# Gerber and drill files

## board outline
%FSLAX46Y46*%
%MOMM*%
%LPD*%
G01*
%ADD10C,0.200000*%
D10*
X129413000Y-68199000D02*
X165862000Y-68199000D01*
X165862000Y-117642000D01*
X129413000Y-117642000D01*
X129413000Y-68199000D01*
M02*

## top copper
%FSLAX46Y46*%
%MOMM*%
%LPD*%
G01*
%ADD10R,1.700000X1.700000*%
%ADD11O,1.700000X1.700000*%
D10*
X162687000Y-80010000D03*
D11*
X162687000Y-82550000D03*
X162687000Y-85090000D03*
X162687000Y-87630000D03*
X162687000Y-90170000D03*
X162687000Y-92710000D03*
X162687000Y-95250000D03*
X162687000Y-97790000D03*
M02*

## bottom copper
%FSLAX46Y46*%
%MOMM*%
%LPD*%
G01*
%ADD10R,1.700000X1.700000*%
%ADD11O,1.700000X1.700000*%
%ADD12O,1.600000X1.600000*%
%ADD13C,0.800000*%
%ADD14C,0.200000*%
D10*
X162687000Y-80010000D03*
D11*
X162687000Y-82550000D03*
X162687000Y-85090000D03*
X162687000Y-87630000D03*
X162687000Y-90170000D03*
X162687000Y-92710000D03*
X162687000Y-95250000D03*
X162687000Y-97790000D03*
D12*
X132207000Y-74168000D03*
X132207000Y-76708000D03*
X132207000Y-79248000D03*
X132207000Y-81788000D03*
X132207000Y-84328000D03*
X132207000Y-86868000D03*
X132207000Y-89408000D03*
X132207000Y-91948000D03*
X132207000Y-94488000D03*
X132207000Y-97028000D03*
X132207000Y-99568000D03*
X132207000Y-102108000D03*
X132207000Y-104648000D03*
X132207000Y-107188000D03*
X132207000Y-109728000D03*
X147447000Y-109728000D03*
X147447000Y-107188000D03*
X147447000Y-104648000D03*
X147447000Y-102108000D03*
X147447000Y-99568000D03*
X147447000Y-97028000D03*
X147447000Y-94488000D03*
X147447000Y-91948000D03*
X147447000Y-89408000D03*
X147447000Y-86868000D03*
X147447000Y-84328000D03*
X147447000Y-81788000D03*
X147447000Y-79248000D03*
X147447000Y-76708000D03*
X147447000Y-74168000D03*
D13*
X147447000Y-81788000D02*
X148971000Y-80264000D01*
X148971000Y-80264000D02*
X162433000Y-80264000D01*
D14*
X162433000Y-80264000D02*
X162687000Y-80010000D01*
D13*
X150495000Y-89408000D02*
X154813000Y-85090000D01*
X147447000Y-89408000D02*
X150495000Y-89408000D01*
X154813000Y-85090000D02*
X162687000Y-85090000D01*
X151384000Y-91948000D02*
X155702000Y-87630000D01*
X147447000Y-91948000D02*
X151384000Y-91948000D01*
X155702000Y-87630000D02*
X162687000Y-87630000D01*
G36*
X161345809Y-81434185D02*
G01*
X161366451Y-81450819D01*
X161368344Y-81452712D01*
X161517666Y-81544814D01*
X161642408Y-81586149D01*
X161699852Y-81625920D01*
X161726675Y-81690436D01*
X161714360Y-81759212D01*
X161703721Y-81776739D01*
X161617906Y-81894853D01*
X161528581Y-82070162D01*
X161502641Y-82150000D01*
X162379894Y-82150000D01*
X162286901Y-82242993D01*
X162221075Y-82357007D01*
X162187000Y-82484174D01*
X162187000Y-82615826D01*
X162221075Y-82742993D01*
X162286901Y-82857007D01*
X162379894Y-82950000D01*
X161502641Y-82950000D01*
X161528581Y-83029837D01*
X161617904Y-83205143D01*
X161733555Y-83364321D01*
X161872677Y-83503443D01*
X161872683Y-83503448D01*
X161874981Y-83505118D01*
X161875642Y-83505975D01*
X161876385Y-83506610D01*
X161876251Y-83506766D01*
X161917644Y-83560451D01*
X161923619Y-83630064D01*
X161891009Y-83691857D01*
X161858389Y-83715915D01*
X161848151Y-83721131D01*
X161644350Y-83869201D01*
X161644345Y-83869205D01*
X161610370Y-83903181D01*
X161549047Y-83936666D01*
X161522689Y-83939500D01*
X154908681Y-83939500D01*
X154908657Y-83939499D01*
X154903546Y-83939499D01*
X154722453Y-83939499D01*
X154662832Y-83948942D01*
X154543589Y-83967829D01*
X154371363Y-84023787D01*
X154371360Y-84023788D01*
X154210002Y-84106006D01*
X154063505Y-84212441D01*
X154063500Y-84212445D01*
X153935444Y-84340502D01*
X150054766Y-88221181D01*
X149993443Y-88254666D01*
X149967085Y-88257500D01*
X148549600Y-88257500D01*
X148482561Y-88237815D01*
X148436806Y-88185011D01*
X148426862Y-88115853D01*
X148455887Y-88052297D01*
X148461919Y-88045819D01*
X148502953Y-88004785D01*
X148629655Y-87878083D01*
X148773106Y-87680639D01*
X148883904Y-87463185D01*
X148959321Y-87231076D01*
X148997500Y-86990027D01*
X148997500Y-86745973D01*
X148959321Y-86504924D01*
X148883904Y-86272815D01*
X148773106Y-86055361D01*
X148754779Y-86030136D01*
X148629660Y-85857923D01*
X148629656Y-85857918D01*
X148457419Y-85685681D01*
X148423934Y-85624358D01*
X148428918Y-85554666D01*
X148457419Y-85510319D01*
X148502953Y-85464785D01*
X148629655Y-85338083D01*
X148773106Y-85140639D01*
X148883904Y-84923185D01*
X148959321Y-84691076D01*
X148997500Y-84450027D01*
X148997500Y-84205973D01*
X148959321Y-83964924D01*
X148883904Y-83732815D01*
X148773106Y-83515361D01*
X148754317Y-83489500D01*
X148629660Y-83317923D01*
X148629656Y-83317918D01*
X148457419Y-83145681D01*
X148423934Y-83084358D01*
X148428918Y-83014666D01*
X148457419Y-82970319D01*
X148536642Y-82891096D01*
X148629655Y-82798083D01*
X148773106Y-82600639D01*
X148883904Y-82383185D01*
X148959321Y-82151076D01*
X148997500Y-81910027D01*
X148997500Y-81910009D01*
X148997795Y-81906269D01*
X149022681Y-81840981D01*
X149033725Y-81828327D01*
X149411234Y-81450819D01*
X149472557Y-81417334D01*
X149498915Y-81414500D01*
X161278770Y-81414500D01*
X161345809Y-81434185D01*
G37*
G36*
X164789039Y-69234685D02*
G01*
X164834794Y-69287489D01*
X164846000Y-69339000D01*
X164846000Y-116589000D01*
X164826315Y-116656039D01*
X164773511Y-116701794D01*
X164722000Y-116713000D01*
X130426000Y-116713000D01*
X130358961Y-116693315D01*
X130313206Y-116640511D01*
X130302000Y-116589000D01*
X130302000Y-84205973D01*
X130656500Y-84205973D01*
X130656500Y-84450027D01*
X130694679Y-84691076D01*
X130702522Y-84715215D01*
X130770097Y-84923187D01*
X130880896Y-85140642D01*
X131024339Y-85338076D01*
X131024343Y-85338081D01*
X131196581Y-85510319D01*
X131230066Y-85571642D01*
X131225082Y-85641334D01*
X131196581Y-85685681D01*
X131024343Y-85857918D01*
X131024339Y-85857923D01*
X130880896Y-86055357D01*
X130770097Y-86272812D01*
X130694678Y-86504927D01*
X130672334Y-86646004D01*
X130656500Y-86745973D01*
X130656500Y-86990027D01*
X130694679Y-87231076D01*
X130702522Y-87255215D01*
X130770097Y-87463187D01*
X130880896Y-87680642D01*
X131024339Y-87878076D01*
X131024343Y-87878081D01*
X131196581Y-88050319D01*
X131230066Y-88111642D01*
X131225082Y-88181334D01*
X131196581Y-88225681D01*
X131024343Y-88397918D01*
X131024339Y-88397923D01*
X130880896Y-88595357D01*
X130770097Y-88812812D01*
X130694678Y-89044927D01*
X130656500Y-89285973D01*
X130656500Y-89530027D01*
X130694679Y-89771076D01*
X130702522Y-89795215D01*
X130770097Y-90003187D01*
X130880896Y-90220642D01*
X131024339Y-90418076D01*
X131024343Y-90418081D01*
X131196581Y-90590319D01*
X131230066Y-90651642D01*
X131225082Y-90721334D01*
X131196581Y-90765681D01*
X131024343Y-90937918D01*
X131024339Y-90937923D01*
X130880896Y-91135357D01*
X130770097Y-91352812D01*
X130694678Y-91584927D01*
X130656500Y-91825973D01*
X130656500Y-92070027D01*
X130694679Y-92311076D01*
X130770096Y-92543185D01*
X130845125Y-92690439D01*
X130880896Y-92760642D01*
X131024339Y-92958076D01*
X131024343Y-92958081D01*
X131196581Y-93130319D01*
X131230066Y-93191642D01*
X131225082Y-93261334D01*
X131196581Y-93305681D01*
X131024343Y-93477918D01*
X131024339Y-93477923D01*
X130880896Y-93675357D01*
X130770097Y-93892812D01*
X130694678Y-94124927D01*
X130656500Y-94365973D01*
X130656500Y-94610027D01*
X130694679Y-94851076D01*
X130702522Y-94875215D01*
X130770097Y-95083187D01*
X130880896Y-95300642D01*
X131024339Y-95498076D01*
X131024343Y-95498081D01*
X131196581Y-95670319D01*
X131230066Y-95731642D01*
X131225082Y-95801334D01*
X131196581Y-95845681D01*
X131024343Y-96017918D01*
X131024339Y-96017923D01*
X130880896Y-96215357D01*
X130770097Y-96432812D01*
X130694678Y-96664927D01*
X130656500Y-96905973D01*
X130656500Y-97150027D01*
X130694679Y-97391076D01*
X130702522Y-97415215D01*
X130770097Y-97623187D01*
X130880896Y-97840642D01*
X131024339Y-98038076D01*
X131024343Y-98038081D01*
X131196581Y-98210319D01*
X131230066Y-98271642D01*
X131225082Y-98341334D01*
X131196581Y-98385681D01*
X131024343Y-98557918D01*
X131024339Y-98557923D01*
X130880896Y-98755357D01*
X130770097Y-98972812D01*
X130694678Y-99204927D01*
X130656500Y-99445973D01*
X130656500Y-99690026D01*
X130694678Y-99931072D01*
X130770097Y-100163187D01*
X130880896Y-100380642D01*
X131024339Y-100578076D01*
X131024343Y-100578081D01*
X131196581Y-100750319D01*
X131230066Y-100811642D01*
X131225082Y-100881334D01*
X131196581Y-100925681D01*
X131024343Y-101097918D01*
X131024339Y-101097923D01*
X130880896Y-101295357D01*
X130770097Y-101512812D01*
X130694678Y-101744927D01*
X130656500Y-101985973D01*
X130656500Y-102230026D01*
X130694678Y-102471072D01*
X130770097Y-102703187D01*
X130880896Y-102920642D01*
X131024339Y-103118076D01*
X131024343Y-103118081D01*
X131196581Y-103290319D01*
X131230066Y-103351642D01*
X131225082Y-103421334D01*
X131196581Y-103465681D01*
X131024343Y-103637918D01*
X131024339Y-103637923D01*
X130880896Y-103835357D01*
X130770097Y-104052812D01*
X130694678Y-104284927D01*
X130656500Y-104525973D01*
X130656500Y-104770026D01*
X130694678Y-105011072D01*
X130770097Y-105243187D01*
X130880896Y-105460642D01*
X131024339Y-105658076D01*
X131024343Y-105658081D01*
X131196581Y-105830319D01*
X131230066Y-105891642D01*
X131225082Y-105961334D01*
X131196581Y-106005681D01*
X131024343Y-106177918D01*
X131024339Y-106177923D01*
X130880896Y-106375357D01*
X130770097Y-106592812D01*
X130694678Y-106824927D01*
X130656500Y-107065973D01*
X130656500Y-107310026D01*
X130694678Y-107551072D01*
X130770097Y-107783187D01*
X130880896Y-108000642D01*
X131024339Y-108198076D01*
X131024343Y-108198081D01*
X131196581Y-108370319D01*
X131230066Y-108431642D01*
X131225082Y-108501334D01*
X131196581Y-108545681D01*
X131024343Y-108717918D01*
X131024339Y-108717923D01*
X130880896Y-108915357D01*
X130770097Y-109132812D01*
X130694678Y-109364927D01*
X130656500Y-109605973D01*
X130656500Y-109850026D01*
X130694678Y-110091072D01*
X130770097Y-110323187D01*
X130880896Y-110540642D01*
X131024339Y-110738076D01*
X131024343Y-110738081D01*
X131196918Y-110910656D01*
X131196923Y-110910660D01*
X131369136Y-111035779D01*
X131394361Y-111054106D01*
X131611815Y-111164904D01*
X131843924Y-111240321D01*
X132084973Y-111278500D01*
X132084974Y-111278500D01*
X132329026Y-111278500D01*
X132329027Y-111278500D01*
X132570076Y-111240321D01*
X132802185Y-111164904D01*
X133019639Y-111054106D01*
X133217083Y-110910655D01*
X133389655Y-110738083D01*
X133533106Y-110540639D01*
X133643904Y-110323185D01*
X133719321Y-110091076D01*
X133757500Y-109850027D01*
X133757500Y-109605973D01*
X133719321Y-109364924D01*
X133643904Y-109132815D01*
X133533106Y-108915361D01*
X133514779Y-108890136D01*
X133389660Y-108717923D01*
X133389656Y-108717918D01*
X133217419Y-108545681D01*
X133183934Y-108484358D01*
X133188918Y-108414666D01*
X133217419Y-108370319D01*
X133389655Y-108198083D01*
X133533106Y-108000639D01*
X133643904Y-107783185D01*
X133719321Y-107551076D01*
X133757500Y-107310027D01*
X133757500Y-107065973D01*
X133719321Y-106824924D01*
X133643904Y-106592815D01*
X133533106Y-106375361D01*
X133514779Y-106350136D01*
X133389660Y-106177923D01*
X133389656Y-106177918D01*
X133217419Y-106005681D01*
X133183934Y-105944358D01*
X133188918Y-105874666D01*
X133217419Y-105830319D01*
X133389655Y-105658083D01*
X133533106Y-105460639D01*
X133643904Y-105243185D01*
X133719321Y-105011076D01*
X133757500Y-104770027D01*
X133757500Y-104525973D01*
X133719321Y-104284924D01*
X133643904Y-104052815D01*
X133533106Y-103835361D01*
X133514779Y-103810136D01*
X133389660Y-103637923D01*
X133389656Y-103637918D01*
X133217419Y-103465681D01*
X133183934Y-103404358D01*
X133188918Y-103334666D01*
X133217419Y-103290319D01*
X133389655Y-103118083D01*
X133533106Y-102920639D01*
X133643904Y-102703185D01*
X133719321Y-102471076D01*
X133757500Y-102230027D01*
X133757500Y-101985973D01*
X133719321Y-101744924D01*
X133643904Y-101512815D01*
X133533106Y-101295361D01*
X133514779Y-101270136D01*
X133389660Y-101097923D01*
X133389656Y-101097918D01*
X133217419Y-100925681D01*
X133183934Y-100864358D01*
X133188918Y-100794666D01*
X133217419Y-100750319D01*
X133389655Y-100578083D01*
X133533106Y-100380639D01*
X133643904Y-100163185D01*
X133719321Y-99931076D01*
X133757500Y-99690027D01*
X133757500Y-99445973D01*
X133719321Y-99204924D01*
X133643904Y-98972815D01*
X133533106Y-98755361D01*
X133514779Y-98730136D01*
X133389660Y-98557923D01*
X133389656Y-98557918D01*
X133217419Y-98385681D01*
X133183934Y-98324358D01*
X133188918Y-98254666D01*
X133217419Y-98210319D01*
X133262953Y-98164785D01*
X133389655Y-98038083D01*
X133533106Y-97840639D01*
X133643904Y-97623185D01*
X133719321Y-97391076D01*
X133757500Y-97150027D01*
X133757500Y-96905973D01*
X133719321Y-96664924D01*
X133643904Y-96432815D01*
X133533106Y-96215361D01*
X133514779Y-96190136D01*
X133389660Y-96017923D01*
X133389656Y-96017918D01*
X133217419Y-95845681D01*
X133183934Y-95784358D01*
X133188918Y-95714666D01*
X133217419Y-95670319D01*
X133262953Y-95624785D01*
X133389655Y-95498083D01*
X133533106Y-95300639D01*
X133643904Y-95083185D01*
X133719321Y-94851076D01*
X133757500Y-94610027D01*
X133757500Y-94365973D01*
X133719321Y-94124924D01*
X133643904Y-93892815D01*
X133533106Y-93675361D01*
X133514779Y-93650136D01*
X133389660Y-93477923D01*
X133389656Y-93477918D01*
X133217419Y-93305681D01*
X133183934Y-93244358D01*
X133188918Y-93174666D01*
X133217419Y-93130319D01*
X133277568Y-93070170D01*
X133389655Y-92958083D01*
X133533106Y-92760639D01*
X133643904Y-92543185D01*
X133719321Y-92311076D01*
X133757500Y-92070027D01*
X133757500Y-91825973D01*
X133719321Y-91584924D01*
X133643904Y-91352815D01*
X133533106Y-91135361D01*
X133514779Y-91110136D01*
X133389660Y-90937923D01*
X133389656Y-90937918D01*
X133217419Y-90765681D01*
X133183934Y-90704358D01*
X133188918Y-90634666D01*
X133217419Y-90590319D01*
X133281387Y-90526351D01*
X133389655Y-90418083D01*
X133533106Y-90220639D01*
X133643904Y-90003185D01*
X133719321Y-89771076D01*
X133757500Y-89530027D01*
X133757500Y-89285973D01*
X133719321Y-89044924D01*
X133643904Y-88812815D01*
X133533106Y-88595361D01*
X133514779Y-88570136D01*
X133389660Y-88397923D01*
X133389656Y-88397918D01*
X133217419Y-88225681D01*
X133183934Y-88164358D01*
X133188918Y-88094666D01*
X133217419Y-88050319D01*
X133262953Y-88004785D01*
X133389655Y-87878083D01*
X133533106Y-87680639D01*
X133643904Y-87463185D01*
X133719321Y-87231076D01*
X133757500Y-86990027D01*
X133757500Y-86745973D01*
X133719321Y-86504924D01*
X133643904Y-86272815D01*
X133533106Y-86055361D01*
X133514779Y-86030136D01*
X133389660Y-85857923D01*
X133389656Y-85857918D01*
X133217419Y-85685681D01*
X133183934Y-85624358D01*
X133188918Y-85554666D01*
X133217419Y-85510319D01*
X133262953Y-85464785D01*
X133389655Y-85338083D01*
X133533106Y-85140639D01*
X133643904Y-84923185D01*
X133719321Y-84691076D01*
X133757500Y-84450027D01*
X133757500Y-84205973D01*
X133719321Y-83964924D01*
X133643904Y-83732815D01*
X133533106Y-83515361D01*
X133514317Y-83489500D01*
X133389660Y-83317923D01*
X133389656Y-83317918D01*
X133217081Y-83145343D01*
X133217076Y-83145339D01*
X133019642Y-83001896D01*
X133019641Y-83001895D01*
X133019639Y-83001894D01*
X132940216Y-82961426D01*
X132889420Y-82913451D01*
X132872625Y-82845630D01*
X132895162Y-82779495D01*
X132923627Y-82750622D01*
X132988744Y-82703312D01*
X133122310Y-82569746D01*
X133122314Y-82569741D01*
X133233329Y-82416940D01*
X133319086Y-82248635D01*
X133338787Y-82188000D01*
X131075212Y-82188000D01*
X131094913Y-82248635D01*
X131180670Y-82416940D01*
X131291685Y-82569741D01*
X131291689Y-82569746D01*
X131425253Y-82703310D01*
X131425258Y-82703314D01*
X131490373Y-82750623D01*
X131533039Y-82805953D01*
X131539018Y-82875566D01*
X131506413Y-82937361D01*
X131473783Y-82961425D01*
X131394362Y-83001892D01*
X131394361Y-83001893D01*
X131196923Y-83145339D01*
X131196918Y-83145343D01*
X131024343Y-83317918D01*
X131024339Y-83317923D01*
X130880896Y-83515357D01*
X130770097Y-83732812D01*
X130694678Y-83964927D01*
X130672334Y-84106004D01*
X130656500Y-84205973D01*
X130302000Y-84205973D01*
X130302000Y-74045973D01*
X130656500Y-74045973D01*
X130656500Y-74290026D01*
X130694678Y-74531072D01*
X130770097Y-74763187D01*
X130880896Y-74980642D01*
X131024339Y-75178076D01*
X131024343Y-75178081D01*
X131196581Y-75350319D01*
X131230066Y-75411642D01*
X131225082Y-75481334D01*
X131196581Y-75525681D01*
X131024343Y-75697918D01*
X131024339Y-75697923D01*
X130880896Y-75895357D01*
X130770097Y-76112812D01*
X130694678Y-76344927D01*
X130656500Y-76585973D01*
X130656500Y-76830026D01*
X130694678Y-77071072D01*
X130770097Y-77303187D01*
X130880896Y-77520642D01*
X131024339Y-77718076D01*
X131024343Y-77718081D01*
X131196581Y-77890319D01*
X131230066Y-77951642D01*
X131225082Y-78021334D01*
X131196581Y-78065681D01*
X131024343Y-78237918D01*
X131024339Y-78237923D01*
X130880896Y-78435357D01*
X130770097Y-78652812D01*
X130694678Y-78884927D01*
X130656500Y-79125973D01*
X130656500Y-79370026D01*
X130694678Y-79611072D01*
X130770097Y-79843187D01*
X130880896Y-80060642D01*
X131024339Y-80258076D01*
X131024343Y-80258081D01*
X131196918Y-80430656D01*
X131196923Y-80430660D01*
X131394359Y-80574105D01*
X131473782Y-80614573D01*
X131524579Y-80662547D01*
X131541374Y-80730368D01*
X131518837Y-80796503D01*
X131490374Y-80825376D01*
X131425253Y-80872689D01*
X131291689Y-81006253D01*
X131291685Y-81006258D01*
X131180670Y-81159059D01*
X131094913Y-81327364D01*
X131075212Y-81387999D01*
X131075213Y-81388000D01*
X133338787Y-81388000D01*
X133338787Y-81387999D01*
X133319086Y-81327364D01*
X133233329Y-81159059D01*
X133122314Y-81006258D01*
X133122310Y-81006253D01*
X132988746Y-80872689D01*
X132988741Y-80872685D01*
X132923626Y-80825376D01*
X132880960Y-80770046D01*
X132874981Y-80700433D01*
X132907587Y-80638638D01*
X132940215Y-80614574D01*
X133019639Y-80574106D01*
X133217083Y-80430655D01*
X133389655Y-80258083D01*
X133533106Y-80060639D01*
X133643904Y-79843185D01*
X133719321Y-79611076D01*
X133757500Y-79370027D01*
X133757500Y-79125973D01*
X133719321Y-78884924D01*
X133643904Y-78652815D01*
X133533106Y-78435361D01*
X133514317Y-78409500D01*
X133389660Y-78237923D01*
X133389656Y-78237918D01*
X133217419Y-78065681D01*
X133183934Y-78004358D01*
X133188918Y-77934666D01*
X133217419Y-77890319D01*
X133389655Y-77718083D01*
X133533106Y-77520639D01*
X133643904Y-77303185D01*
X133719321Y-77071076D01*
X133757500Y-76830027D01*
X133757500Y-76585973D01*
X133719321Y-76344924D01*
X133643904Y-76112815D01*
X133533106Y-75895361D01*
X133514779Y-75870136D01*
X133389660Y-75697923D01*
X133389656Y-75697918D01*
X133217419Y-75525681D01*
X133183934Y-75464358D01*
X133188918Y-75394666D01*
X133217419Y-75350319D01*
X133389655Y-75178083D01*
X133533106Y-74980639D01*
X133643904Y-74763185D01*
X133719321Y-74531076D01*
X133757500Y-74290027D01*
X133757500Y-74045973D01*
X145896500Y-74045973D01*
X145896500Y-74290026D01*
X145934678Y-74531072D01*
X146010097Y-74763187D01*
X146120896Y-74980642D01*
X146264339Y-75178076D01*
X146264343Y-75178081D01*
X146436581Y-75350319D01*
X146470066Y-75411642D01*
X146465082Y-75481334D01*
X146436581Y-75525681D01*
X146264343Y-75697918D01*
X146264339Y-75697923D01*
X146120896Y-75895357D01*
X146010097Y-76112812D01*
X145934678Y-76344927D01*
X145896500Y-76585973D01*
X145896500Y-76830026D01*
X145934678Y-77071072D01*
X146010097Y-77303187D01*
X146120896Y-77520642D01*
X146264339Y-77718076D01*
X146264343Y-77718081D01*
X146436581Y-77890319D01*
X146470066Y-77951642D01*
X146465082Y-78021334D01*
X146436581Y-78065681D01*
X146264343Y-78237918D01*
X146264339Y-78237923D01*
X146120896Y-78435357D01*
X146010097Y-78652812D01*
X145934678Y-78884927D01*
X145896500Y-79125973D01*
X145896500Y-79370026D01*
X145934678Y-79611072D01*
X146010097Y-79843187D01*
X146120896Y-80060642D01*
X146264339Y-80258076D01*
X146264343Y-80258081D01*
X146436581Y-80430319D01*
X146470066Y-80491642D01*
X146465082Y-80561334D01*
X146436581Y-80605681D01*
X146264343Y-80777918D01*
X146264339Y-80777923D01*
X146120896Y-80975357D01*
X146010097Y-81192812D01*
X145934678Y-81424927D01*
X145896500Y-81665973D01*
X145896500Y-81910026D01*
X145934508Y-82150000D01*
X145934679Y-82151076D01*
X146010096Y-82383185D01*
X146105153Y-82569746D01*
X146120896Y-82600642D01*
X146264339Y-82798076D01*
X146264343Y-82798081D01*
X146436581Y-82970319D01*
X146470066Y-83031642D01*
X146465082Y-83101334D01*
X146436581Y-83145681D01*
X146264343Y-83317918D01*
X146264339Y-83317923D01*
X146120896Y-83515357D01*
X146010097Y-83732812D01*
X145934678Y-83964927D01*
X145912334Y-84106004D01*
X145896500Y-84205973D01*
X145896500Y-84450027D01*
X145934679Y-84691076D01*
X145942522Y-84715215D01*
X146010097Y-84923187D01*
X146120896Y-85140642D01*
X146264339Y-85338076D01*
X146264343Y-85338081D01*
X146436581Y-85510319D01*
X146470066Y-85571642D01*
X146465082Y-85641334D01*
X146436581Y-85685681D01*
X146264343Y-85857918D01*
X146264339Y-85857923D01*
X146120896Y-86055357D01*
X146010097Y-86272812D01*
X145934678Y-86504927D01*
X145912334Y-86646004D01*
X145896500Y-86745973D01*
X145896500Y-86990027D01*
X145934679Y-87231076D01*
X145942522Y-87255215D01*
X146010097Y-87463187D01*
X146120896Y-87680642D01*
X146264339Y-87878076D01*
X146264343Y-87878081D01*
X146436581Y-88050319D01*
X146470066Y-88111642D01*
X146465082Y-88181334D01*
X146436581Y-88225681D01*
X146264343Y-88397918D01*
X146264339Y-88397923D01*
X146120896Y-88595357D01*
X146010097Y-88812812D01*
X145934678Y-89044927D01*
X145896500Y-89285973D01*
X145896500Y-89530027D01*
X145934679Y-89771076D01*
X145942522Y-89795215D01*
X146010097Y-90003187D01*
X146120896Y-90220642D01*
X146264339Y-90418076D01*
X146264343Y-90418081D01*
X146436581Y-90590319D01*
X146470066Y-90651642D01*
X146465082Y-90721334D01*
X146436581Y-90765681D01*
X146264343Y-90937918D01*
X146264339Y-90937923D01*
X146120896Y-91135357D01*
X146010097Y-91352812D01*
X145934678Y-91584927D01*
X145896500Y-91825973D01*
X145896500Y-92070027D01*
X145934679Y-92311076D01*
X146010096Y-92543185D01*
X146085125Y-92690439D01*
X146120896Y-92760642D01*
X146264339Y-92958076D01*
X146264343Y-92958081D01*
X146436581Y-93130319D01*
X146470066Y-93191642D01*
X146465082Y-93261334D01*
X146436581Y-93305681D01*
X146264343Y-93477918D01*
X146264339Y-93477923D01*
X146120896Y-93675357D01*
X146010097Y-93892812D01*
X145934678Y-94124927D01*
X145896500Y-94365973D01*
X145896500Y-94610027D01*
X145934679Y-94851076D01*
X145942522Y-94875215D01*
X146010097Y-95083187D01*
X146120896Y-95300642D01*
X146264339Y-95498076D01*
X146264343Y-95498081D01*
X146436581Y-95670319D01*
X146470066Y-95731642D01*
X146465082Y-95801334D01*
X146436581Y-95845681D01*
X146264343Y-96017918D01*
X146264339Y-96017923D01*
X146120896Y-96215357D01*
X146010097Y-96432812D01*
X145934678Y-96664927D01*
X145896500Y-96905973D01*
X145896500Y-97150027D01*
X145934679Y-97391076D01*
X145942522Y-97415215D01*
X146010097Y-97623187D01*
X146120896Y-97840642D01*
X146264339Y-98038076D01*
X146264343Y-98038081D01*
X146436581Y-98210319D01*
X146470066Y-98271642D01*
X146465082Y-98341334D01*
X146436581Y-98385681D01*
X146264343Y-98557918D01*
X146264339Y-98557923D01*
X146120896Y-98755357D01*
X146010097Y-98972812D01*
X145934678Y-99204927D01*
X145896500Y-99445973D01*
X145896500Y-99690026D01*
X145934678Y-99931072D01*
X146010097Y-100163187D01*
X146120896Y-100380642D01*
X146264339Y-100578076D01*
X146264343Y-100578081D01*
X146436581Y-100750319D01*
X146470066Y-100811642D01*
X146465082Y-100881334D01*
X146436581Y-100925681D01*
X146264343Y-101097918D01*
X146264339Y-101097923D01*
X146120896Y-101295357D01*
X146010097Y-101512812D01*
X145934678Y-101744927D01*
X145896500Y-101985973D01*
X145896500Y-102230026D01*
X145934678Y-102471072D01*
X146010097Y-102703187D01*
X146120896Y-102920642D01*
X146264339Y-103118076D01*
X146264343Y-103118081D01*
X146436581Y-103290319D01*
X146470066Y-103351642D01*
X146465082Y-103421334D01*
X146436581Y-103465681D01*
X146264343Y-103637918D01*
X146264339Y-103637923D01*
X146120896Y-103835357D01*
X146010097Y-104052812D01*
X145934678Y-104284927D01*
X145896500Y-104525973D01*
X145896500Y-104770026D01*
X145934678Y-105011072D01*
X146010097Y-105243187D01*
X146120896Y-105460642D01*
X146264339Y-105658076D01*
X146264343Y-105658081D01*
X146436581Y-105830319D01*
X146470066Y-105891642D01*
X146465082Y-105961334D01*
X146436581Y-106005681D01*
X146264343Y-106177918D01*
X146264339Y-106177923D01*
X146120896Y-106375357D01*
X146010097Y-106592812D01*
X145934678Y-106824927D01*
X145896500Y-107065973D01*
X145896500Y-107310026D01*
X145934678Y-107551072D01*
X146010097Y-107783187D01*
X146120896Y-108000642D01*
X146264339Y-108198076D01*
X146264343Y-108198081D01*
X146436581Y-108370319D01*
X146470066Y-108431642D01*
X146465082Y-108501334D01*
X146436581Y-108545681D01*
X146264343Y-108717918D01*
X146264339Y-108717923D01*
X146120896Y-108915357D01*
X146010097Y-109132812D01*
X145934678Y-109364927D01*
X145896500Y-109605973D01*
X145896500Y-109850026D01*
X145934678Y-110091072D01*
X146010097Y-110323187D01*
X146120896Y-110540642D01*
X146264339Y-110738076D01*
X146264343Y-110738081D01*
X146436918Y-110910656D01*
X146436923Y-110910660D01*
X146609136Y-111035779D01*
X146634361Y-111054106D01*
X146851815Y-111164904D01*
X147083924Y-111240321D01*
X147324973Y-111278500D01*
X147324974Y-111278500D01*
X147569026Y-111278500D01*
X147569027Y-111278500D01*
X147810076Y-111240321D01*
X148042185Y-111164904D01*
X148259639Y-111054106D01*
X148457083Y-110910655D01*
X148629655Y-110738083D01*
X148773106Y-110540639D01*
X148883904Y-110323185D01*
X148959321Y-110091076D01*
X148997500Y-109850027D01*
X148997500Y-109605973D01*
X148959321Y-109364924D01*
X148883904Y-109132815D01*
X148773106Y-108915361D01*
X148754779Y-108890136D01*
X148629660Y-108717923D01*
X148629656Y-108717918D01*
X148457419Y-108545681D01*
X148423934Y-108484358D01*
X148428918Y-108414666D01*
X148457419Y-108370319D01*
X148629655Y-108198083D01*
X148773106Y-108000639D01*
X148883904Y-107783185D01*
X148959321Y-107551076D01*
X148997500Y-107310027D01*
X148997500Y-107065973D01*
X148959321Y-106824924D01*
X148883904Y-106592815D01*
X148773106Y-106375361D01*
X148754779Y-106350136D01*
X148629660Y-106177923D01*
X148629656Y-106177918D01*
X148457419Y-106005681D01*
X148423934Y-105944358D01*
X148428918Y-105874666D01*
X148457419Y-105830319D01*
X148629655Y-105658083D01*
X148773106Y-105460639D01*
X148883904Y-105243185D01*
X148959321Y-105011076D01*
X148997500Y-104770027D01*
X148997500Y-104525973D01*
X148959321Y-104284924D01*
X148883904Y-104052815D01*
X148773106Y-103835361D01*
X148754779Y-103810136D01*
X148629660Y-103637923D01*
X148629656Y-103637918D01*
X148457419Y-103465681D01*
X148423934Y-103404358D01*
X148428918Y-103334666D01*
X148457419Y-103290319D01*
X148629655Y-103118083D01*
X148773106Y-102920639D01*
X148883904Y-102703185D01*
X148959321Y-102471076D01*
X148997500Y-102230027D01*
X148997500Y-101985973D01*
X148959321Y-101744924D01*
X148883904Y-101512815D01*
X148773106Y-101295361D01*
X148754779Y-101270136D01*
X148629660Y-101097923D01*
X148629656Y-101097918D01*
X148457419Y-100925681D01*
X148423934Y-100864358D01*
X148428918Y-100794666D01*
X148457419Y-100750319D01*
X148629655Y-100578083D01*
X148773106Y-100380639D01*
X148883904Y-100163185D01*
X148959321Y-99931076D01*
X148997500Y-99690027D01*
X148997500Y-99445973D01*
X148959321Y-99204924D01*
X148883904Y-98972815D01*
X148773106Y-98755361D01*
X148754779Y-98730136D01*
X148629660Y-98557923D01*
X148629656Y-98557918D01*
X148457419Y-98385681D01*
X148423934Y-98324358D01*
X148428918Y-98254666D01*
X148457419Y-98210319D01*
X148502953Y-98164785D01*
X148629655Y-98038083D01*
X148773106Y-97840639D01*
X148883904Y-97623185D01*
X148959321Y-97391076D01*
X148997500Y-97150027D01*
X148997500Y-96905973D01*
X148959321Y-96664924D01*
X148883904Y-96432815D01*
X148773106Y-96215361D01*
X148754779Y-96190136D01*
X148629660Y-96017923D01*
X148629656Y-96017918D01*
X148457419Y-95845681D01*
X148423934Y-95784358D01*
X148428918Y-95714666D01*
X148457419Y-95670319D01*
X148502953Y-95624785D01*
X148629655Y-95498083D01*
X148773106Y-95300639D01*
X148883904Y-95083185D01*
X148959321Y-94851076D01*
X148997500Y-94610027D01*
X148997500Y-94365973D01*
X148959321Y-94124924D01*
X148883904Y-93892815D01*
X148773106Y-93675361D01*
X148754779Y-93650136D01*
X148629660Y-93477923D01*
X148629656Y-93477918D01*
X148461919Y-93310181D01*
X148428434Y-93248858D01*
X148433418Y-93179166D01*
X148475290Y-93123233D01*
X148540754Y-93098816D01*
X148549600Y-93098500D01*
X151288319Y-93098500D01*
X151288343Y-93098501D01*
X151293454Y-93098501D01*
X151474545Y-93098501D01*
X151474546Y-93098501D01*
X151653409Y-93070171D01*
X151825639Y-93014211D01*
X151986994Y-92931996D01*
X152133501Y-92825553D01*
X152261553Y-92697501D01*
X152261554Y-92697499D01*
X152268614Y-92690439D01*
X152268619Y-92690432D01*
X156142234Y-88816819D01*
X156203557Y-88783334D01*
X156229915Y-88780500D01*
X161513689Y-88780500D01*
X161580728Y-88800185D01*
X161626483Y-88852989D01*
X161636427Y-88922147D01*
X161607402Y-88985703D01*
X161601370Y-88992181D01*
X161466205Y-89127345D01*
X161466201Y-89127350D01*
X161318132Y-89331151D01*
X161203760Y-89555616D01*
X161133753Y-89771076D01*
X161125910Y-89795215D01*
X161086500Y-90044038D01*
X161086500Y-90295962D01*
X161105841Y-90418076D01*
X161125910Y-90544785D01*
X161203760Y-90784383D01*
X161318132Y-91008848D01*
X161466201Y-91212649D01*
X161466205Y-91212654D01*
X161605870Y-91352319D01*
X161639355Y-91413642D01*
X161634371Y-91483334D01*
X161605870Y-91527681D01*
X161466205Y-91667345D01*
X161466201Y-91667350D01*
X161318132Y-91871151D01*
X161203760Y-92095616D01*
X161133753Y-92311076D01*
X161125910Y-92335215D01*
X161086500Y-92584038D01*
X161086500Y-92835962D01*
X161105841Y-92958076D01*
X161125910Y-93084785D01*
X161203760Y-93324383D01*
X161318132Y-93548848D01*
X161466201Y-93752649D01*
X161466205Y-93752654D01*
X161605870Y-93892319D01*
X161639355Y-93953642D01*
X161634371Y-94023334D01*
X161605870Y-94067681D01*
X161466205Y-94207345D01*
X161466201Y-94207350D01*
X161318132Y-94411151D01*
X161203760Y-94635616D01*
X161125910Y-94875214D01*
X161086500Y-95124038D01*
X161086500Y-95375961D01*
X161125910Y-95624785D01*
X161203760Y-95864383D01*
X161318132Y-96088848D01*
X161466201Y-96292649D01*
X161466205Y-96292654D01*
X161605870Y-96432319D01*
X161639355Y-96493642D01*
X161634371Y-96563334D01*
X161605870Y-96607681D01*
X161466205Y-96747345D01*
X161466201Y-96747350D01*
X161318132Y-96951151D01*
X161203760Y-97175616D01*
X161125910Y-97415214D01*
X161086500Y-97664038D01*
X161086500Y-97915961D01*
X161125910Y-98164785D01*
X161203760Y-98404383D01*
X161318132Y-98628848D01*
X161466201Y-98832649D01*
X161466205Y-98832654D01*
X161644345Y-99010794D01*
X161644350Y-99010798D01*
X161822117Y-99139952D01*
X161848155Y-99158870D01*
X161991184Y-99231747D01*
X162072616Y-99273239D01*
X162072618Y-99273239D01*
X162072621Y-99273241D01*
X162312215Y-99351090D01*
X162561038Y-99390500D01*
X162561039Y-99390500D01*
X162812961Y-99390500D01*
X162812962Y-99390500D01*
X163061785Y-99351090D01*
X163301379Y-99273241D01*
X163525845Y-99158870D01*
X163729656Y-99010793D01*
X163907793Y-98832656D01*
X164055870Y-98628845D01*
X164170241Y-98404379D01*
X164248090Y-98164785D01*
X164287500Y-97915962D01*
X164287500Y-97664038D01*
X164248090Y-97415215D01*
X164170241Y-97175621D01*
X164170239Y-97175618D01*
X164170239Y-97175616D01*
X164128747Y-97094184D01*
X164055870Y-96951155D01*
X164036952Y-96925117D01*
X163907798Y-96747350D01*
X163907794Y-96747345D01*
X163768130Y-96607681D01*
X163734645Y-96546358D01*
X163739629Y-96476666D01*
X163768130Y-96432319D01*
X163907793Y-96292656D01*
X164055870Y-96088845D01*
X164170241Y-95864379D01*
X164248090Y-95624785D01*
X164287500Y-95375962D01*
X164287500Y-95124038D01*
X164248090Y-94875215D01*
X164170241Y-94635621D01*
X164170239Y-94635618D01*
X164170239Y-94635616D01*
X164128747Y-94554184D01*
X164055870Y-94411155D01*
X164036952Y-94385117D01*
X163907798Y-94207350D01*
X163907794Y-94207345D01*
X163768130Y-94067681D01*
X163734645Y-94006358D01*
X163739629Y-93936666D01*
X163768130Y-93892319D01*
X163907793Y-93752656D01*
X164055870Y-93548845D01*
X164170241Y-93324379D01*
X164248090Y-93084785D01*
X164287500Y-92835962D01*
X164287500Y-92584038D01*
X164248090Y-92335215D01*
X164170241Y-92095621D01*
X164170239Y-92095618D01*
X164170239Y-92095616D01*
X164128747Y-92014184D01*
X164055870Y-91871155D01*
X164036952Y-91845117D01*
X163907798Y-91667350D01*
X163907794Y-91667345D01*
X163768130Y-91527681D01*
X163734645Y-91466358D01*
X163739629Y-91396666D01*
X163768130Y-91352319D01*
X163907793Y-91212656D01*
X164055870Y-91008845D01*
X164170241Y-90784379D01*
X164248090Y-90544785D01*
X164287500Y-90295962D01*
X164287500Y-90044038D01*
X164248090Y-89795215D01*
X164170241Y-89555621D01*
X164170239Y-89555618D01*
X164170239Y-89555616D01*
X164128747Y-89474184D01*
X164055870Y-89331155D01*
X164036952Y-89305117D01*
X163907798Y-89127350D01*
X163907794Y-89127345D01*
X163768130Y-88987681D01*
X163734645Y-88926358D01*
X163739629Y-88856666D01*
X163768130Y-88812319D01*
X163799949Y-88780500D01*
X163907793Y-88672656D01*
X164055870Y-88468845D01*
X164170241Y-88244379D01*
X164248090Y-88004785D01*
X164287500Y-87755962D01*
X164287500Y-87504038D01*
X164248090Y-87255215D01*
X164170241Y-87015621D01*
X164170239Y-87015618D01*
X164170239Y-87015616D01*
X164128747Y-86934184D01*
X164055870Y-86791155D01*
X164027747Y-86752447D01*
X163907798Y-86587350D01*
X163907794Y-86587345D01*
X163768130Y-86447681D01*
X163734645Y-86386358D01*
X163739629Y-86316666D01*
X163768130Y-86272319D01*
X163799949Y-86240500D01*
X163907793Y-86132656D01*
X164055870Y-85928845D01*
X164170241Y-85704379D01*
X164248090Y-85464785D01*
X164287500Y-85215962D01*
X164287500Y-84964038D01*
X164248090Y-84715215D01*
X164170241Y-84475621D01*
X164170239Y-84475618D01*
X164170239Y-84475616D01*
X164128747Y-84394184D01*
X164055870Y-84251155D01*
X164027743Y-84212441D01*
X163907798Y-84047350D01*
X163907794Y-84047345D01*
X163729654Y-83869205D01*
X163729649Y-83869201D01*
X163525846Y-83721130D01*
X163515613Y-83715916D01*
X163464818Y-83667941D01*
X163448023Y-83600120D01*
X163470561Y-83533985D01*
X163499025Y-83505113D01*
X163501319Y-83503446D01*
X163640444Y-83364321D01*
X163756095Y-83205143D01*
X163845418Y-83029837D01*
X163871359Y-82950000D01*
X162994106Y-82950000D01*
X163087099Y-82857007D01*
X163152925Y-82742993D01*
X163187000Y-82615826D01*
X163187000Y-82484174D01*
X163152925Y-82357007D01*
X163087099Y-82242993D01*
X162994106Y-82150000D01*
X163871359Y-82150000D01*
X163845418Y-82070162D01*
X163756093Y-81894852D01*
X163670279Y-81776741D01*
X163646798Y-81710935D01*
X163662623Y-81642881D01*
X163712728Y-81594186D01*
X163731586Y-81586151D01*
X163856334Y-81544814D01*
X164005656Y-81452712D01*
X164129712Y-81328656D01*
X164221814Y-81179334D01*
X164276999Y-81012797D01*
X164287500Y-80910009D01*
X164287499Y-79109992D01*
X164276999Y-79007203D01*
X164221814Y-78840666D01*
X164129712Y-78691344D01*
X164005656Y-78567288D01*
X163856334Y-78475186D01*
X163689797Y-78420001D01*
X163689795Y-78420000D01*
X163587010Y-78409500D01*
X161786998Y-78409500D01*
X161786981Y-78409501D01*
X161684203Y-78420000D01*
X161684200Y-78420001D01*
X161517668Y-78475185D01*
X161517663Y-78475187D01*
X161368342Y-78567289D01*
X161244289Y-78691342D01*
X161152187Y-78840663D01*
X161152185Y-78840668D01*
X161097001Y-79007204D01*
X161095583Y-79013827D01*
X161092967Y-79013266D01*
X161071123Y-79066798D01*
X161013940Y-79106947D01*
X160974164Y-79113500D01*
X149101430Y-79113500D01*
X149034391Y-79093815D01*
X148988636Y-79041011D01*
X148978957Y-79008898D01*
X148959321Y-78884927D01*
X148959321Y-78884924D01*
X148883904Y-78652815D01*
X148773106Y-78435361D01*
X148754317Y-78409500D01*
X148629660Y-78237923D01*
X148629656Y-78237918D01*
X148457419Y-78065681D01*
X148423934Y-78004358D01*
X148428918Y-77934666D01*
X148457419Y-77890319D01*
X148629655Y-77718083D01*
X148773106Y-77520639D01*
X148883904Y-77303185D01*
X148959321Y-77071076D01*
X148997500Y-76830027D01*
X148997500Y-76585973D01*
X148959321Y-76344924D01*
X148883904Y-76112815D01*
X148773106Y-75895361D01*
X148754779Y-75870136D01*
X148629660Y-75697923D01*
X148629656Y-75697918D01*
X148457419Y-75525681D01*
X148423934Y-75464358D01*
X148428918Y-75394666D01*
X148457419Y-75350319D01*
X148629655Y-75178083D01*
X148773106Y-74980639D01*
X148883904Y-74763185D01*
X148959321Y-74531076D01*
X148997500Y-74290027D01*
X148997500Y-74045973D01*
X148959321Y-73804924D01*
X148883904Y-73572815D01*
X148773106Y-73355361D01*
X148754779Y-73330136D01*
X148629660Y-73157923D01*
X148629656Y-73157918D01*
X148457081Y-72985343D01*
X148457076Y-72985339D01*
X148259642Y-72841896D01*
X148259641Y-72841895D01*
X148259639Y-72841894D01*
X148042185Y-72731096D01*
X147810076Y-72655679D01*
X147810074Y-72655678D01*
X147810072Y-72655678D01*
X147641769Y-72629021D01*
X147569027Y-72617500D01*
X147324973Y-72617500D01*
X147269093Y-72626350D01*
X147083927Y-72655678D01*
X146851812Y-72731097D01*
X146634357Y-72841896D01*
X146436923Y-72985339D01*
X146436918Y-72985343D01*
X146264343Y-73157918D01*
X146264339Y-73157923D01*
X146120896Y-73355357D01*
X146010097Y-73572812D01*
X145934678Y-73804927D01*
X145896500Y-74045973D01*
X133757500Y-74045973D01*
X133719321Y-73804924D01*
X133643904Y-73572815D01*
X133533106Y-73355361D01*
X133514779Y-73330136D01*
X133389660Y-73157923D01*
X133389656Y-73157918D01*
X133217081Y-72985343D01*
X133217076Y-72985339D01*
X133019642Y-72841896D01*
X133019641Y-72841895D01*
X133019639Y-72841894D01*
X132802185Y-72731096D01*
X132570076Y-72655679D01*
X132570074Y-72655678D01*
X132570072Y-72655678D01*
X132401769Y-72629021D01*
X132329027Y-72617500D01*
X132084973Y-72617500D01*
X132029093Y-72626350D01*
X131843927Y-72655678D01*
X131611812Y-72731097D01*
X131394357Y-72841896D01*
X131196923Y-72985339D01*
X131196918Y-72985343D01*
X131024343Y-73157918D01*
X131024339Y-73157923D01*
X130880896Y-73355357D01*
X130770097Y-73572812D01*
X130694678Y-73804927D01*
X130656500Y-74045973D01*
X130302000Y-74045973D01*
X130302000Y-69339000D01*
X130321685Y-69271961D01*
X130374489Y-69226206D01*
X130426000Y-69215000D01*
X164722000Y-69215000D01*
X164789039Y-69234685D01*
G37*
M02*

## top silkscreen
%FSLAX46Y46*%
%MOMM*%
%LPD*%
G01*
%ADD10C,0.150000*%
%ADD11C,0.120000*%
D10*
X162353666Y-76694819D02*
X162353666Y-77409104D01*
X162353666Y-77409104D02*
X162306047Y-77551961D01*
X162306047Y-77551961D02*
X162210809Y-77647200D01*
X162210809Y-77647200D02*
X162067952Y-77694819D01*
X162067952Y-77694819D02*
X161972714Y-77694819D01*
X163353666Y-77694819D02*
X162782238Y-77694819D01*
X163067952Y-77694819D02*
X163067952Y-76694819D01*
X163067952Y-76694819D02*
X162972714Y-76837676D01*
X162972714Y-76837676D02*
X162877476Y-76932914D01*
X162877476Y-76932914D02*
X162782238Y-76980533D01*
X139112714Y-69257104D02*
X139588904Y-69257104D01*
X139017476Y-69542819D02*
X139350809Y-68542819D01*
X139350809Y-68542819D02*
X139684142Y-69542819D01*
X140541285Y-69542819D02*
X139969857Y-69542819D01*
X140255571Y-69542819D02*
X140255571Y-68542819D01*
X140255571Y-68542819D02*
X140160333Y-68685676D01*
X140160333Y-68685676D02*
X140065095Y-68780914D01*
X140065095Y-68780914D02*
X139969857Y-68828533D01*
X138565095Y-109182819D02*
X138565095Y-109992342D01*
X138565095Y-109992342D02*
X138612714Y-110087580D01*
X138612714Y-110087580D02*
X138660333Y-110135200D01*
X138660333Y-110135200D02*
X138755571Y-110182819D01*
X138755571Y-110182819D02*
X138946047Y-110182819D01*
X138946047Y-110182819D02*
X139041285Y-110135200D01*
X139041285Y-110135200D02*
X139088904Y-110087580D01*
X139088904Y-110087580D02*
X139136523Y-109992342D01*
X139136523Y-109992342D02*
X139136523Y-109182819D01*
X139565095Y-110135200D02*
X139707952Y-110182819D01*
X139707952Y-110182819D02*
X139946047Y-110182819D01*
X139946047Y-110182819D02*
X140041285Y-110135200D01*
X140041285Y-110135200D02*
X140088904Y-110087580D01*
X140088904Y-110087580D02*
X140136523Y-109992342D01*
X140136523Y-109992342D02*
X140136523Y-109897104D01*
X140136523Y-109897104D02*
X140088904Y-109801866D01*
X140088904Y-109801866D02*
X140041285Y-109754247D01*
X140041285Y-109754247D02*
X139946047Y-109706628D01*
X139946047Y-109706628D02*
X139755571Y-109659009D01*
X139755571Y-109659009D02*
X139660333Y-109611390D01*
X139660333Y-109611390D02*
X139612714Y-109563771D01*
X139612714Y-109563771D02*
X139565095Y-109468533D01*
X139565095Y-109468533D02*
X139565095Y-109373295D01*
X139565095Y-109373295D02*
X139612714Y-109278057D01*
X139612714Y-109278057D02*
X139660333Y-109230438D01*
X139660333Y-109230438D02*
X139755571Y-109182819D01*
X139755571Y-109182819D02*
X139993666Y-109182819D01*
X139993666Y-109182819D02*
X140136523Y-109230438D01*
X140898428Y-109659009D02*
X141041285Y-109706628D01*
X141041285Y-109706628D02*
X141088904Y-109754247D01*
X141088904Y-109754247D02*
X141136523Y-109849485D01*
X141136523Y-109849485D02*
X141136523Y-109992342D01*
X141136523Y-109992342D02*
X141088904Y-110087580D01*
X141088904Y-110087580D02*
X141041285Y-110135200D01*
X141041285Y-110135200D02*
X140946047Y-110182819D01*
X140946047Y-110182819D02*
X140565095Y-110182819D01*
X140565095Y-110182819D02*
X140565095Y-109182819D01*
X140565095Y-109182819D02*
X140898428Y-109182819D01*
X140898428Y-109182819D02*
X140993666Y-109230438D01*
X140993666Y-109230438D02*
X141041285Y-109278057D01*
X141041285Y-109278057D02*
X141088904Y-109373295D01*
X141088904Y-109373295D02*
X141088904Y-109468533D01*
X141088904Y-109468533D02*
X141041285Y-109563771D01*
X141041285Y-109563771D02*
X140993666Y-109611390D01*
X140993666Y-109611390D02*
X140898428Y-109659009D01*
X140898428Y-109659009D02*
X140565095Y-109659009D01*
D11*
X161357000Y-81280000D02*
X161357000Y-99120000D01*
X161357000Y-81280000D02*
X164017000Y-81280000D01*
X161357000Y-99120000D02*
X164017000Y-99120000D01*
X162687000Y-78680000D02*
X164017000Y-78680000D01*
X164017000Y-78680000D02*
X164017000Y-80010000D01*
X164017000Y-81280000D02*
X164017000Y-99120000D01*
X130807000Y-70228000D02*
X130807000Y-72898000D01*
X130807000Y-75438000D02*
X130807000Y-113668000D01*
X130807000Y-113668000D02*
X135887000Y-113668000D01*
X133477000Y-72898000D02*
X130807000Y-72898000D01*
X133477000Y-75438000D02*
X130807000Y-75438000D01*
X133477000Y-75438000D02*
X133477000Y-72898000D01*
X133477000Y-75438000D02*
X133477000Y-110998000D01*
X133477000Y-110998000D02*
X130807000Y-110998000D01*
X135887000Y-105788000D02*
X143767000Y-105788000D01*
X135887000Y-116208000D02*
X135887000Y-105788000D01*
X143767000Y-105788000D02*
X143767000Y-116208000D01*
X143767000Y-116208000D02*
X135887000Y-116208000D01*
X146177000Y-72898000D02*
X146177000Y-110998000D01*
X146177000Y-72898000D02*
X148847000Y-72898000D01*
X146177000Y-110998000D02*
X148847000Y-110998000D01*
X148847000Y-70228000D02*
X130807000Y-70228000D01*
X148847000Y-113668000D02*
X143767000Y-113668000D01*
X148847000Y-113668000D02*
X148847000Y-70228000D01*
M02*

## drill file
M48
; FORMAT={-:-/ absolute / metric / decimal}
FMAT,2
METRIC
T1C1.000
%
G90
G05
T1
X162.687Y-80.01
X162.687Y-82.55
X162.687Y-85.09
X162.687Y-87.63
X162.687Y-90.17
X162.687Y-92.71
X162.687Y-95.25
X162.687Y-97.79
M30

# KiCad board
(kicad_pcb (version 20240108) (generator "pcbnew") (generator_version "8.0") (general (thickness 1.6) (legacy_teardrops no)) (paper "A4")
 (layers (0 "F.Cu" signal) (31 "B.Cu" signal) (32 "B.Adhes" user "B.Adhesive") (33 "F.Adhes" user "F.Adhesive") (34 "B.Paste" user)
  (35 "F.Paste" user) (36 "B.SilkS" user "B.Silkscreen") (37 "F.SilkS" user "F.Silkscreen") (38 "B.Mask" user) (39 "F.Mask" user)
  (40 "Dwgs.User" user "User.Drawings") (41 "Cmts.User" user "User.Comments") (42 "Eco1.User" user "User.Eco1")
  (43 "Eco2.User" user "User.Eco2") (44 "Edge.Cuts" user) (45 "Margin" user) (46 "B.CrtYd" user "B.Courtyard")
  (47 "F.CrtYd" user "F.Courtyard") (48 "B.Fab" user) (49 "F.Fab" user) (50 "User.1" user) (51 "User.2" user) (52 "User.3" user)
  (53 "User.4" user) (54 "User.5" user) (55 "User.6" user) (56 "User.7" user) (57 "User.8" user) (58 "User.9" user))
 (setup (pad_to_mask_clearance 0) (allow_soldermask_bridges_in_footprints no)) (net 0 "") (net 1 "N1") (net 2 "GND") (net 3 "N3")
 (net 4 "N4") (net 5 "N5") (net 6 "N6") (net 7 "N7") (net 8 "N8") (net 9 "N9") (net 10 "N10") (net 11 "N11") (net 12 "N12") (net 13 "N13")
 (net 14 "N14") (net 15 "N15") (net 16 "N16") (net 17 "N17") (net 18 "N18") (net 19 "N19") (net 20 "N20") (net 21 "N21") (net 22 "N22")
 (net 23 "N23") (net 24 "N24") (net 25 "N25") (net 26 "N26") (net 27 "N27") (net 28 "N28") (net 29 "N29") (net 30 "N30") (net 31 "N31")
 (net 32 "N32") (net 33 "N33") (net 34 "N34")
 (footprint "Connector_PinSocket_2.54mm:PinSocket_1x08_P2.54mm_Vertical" (layer "F.Cu") (at 162.687 80.01)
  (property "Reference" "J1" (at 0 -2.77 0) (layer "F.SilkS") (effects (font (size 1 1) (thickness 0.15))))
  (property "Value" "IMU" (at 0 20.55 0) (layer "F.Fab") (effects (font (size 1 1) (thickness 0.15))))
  (fp_line (start -1.33 1.27) (end -1.33 19.11) (stroke (width 0.12) (type solid)) (layer "F.SilkS"))
  (fp_line (start -1.33 1.27) (end 1.33 1.27) (stroke (width 0.12) (type solid)) (layer "F.SilkS"))
  (fp_line (start -1.33 19.11) (end 1.33 19.11) (stroke (width 0.12) (type solid)) (layer "F.SilkS"))
  (fp_line (start 0 -1.33) (end 1.33 -1.33) (stroke (width 0.12) (type solid)) (layer "F.SilkS"))
  (fp_line (start 1.33 -1.33) (end 1.33 0) (stroke (width 0.12) (type solid)) (layer "F.SilkS"))
  (fp_line (start 1.33 1.27) (end 1.33 19.11) (stroke (width 0.12) (type solid)) (layer "F.SilkS"))
  (pad "1" thru_hole rect (at 0 0) (size 1.7 1.7) (drill 1) (layers "*.Cu" "*.Mask") (remove_unused_layers no) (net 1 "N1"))
  (pad "2" thru_hole oval (at 0 2.54) (size 1.7 1.7) (drill 1) (layers "*.Cu" "*.Mask") (remove_unused_layers no) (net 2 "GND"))
  (pad "3" thru_hole oval (at 0 5.08) (size 1.7 1.7) (drill 1) (layers "*.Cu" "*.Mask") (remove_unused_layers no) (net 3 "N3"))
  (pad "4" thru_hole oval (at 0 7.62) (size 1.7 1.7) (drill 1) (layers "*.Cu" "*.Mask") (remove_unused_layers no) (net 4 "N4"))
  (pad "5" thru_hole oval (at 0 10.16) (size 1.7 1.7) (drill 1) (layers "*.Cu" "*.Mask") (remove_unused_layers no) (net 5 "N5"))
  (pad "6" thru_hole oval (at 0 12.7) (size 1.7 1.7) (drill 1) (layers "*.Cu" "*.Mask") (remove_unused_layers no) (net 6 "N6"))
  (pad "7" thru_hole oval (at 0 15.24) (size 1.7 1.7) (drill 1) (layers "*.Cu" "*.Mask") (remove_unused_layers no) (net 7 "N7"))
  (pad "8" thru_hole oval (at 0 17.78) (size 1.7 1.7) (drill 1) (layers "*.Cu" "*.Mask") (remove_unused_layers no) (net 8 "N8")))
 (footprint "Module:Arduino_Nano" (layer "F.Cu") (at 132.207 74.168)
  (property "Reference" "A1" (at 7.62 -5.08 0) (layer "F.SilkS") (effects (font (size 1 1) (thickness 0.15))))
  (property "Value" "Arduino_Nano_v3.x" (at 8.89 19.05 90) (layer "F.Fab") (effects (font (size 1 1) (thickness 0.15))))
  (fp_line (start -1.4 -3.94) (end -1.4 -1.27) (stroke (width 0.12) (type solid)) (layer "F.SilkS"))
  (fp_line (start -1.4 1.27) (end -1.4 39.5) (stroke (width 0.12) (type solid)) (layer "F.SilkS"))
  (fp_line (start -1.4 39.5) (end 3.68 39.5) (stroke (width 0.12) (type solid)) (layer "F.SilkS"))
  (fp_line (start 1.27 -1.27) (end -1.4 -1.27) (stroke (width 0.12) (type solid)) (layer "F.SilkS"))
  (fp_line (start 1.27 1.27) (end -1.4 1.27) (stroke (width 0.12) (type solid)) (layer "F.SilkS"))
  (fp_line (start 1.27 1.27) (end 1.27 -1.27) (stroke (width 0.12) (type solid)) (layer "F.SilkS"))
  (fp_line (start 1.27 1.27) (end 1.27 36.83) (stroke (width 0.12) (type solid)) (layer "F.SilkS"))
  (fp_line (start 1.27 36.83) (end -1.4 36.83) (stroke (width 0.12) (type solid)) (layer "F.SilkS"))
  (fp_line (start 3.68 31.62) (end 11.56 31.62) (stroke (width 0.12) (type solid)) (layer "F.SilkS"))
  (fp_line (start 3.68 42.04) (end 3.68 31.62) (stroke (width 0.12) (type solid)) (layer "F.SilkS"))
  (fp_line (start 11.56 31.62) (end 11.56 42.04) (stroke (width 0.12) (type solid)) (layer "F.SilkS"))
  (fp_line (start 11.56 42.04) (end 3.68 42.04) (stroke (width 0.12) (type solid)) (layer "F.SilkS"))
  (fp_line (start 13.97 -1.27) (end 13.97 36.83) (stroke (width 0.12) (type solid)) (layer "F.SilkS"))
  (fp_line (start 13.97 -1.27) (end 16.64 -1.27) (stroke (width 0.12) (type solid)) (layer "F.SilkS"))
  (fp_line (start 13.97 36.83) (end 16.64 36.83) (stroke (width 0.12) (type solid)) (layer "F.SilkS"))
  (fp_line (start 16.64 -3.94) (end -1.4 -3.94) (stroke (width 0.12) (type solid)) (layer "F.SilkS"))
  (fp_line (start 16.64 39.5) (end 11.56 39.5) (stroke (width 0.12) (type solid)) (layer "F.SilkS"))
  (fp_line (start 16.64 39.5) (end 16.64 -3.94) (stroke (width 0.12) (type solid)) (layer "F.SilkS"))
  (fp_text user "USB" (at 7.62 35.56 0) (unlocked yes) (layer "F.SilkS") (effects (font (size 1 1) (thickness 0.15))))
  (pad "1" smd oval (at 0 0) (size 1.6 1.6) (layers "B.Cu" "B.Paste" "B.Mask") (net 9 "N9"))
  (pad "2" smd oval (at 0 2.54) (size 1.6 1.6) (layers "B.Cu" "B.Paste" "B.Mask") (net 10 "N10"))
  (pad "3" smd oval (at 0 5.08) (size 1.6 1.6) (layers "B.Cu" "B.Paste" "B.Mask") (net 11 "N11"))
  (pad "4" smd oval (at 0 7.62) (size 1.6 1.6) (layers "B.Cu" "B.Paste" "B.Mask") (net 2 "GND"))
  (pad "5" smd oval (at 0 10.16) (size 1.6 1.6) (layers "B.Cu" "B.Paste" "B.Mask") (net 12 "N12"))
  (pad "6" smd oval (at 0 12.7) (size 1.6 1.6) (layers "B.Cu" "B.Paste" "B.Mask") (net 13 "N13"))
  (pad "7" smd oval (at 0 15.24) (size 1.6 1.6) (layers "B.Cu" "B.Paste" "B.Mask") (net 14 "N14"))
  (pad "8" smd oval (at 0 17.78) (size 1.6 1.6) (layers "B.Cu" "B.Paste" "B.Mask") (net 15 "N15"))
  (pad "9" smd oval (at 0 20.32) (size 1.6 1.6) (layers "B.Cu" "B.Paste" "B.Mask") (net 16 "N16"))
  (pad "10" smd oval (at 0 22.86) (size 1.6 1.6) (layers "B.Cu" "B.Paste" "B.Mask") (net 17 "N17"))
  (pad "11" smd oval (at 0 25.4) (size 1.6 1.6) (layers "B.Cu" "B.Paste" "B.Mask") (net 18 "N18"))
  (pad "12" smd oval (at 0 27.94) (size 1.6 1.6) (layers "B.Cu" "B.Paste" "B.Mask") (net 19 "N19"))
  (pad "13" smd oval (at 0 30.48) (size 1.6 1.6) (layers "B.Cu" "B.Paste" "B.Mask") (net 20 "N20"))
  (pad "14" smd oval (at 0 33.02) (size 1.6 1.6) (layers "B.Cu" "B.Paste" "B.Mask") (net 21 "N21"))
  (pad "15" smd oval (at 0 35.56) (size 1.6 1.6) (layers "B.Cu" "B.Paste" "B.Mask") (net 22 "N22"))
  (pad "16" smd oval (at 15.24 35.56) (size 1.6 1.6) (layers "B.Cu" "B.Paste" "B.Mask") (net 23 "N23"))
  (pad "17" smd oval (at 15.24 33.02) (size 1.6 1.6) (layers "B.Cu" "B.Paste" "B.Mask") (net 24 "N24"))
  (pad "18" smd oval (at 15.24 30.48) (size 1.6 1.6) (layers "B.Cu" "B.Paste" "B.Mask") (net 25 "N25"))
  (pad "19" smd oval (at 15.24 27.94) (size 1.6 1.6) (layers "B.Cu" "B.Paste" "B.Mask") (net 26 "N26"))
  (pad "20" smd oval (at 15.24 25.4) (size 1.6 1.6) (layers "B.Cu" "B.Paste" "B.Mask") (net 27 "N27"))
  (pad "21" smd oval (at 15.24 22.86) (size 1.6 1.6) (layers "B.Cu" "B.Paste" "B.Mask") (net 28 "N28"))
  (pad "22" smd oval (at 15.24 20.32) (size 1.6 1.6) (layers "B.Cu" "B.Paste" "B.Mask") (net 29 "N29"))
  (pad "23" smd oval (at 15.24 17.78) (size 1.6 1.6) (layers "B.Cu" "B.Paste" "B.Mask") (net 4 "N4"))
  (pad "24" smd oval (at 15.24 15.24) (size 1.6 1.6) (layers "B.Cu" "B.Paste" "B.Mask") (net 3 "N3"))
  (pad "25" smd oval (at 15.24 12.7) (size 1.6 1.6) (layers "B.Cu" "B.Paste" "B.Mask") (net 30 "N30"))
  (pad "26" smd oval (at 15.24 10.16) (size 1.6 1.6) (layers "B.Cu" "B.Paste" "B.Mask") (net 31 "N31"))
  (pad "27" smd oval (at 15.24 7.62) (size 1.6 1.6) (layers "B.Cu" "B.Paste" "B.Mask") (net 1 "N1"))
  (pad "28" smd oval (at 15.24 5.08) (size 1.6 1.6) (layers "B.Cu" "B.Paste" "B.Mask") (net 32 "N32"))
  (pad "29" smd oval (at 15.24 2.54) (size 1.6 1.6) (layers "B.Cu" "B.Paste" "B.Mask") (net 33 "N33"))
  (pad "30" smd oval (at 15.24 0) (size 1.6 1.6) (layers "B.Cu" "B.Paste" "B.Mask") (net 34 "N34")))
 (gr_rect (start 129.413 68.199) (end 165.862 117.642) (stroke (width 0.2) (type default)) (fill none) (layer "Edge.Cuts"))
 (segment (start 147.447 81.788) (end 148.971 80.264) (width 0.8) (layer "B.Cu") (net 1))
 (segment (start 148.971 80.264) (end 162.433 80.264) (width 0.8) (layer "B.Cu") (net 1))
 (segment (start 162.433 80.264) (end 162.687 80.01) (width 0.2) (layer "B.Cu") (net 1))
 (segment (start 150.495 89.408) (end 154.813 85.09) (width 0.8) (layer "B.Cu") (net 3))
 (segment (start 147.447 89.408) (end 150.495 89.408) (width 0.8) (layer "B.Cu") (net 3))
 (segment (start 154.813 85.09) (end 162.687 85.09) (width 0.8) (layer "B.Cu") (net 3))
 (segment (start 151.384 91.948) (end 155.702 87.63) (width 0.8) (layer "B.Cu") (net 4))
 (segment (start 147.447 91.948) (end 151.384 91.948) (width 0.8) (layer "B.Cu") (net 4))
 (segment (start 155.702 87.63) (end 162.687 87.63) (width 0.8) (layer "B.Cu") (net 4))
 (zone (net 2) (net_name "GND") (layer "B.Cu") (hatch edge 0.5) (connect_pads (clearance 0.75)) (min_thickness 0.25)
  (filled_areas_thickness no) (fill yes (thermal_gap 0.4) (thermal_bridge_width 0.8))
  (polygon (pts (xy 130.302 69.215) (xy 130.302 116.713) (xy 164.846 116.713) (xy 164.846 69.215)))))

